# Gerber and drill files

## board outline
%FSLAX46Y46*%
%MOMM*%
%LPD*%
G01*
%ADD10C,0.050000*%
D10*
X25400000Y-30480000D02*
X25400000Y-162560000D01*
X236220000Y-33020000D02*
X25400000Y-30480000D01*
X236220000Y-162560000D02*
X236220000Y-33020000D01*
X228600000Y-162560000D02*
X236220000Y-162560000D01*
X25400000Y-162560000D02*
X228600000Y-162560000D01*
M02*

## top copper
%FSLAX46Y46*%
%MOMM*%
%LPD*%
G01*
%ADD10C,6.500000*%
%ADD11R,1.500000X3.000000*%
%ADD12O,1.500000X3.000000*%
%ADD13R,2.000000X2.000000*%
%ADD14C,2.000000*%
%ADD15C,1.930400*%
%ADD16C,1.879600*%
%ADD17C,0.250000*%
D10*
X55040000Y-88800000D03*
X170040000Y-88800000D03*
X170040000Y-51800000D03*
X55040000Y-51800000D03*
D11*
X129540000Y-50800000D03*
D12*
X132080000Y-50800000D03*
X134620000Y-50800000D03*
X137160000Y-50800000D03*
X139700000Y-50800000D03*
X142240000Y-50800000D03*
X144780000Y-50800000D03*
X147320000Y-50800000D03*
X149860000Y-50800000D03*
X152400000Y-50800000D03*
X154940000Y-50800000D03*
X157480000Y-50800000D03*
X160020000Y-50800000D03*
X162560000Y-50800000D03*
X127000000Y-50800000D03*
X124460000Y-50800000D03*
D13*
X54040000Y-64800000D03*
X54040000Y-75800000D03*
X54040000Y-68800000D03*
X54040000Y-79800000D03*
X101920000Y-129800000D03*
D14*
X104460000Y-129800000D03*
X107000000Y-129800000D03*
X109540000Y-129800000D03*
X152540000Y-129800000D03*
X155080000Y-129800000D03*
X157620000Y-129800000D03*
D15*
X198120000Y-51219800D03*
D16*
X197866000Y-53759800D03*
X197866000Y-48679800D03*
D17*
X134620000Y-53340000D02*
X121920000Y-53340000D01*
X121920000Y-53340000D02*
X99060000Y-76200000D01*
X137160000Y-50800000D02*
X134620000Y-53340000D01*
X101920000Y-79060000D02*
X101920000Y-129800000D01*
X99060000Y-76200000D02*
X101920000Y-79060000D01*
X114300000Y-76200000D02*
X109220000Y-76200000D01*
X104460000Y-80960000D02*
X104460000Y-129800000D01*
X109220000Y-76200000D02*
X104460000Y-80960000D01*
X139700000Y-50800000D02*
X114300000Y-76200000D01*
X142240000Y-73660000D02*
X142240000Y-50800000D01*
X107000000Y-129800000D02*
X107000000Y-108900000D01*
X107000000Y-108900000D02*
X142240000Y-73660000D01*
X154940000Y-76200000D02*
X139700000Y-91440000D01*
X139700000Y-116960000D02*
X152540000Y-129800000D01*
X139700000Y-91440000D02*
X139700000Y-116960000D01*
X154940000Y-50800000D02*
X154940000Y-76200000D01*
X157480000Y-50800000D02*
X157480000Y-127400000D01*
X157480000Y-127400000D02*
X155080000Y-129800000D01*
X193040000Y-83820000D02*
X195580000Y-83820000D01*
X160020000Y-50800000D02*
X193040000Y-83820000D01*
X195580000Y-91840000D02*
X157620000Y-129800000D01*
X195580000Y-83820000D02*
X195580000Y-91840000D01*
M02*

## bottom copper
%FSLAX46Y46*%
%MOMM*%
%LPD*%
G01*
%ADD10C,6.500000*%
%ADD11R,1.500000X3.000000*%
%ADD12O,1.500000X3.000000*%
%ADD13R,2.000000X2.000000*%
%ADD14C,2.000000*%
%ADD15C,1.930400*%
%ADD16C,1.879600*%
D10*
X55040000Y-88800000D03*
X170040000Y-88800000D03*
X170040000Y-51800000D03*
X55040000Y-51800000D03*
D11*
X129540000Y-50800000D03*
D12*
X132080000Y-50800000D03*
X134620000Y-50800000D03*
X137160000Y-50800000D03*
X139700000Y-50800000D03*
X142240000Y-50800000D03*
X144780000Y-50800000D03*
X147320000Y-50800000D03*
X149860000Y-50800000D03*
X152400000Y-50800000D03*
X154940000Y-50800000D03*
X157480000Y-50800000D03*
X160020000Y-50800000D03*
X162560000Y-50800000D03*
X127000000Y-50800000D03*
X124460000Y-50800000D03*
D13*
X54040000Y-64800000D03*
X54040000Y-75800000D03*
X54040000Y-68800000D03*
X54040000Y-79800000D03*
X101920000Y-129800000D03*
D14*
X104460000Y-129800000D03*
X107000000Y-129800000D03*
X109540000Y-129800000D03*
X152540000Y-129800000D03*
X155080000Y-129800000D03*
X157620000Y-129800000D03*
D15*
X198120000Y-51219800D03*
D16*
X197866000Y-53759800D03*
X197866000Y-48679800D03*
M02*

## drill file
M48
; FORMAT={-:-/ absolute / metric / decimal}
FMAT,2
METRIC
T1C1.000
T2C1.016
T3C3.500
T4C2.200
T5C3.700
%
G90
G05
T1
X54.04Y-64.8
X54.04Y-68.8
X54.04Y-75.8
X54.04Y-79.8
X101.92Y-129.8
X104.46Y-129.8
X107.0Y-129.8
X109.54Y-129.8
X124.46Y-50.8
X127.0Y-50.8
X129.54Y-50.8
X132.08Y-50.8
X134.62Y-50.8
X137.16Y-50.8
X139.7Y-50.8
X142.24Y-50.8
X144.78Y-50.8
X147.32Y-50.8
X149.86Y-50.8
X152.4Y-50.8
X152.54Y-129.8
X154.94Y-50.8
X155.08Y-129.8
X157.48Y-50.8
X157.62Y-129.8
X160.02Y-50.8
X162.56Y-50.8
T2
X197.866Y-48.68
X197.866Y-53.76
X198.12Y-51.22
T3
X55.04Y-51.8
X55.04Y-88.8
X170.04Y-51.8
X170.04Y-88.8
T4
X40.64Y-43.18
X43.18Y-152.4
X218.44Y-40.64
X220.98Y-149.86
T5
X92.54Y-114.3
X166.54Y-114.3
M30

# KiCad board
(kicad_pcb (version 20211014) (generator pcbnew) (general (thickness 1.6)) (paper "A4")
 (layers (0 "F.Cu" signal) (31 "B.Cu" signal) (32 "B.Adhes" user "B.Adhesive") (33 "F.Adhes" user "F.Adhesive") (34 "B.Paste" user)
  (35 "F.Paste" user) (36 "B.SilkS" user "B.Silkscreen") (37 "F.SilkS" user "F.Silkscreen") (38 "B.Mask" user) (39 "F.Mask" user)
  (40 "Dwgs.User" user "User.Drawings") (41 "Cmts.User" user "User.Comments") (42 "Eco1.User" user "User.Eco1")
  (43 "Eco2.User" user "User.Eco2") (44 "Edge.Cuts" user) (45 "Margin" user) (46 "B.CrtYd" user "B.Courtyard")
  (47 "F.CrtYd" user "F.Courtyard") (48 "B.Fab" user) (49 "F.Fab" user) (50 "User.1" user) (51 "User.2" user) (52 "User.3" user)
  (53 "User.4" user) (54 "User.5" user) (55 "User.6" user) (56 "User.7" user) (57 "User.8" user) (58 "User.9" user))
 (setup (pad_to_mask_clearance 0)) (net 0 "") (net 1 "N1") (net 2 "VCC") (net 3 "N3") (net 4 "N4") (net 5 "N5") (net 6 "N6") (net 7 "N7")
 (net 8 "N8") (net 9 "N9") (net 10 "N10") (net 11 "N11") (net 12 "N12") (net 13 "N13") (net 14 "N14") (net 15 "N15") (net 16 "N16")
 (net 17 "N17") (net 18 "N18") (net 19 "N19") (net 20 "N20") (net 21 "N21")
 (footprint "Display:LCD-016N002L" (layer "F.Cu") (at 129.54 50.8)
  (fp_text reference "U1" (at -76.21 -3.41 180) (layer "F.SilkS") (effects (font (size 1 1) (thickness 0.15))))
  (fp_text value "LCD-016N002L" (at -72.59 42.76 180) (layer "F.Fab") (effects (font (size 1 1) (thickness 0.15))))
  (pad "" thru_hole circle (at -74.5 38 180) (size 6.5 6.5) (drill 3.5) (layers *.Cu *.Mask))
  (pad "" thru_hole circle (at 40.5 38 180) (size 6.5 6.5) (drill 3.5) (layers *.Cu *.Mask))
  (pad "" thru_hole circle (at 40.5 1 180) (size 6.5 6.5) (drill 3.5) (layers *.Cu *.Mask))
  (pad "" thru_hole circle (at -74.5 1 180) (size 6.5 6.5) (drill 3.5) (layers *.Cu *.Mask))
  (pad "1" thru_hole rect (at 0 0 180) (size 1.5 3) (drill 1) (layers *.Cu *.Mask) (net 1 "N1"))
  (pad "2" thru_hole oval (at 2.54 0 180) (size 1.5 3) (drill 1) (layers *.Cu *.Mask) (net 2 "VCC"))
  (pad "3" thru_hole oval (at 5.08 0 180) (size 1.5 3) (drill 1) (layers *.Cu *.Mask) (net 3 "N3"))
  (pad "4" thru_hole oval (at 7.62 0 180) (size 1.5 3) (drill 1) (layers *.Cu *.Mask) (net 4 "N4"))
  (pad "5" thru_hole oval (at 10.16 0 180) (size 1.5 3) (drill 1) (layers *.Cu *.Mask) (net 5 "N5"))
  (pad "6" thru_hole oval (at 12.7 0 180) (size 1.5 3) (drill 1) (layers *.Cu *.Mask) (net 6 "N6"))
  (pad "7" thru_hole oval (at 15.24 0 180) (size 1.5 3) (drill 1) (layers *.Cu *.Mask) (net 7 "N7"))
  (pad "8" thru_hole oval (at 17.78 0 180) (size 1.5 3) (drill 1) (layers *.Cu *.Mask) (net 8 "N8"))
  (pad "9" thru_hole oval (at 20.32 0 180) (size 1.5 3) (drill 1) (layers *.Cu *.Mask) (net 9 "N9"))
  (pad "10" thru_hole oval (at 22.86 0 180) (size 1.5 3) (drill 1) (layers *.Cu *.Mask) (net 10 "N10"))
  (pad "11" thru_hole oval (at 25.4 0 180) (size 1.5 3) (drill 1) (layers *.Cu *.Mask) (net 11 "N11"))
  (pad "12" thru_hole oval (at 27.94 0 180) (size 1.5 3) (drill 1) (layers *.Cu *.Mask) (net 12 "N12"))
  (pad "13" thru_hole oval (at 30.48 0 180) (size 1.5 3) (drill 1) (layers *.Cu *.Mask) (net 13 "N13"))
  (pad "14" thru_hole oval (at 33.02 0 180) (size 1.5 3) (drill 1) (layers *.Cu *.Mask) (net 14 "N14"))
  (pad "15" thru_hole oval (at -2.54 0 180) (size 1.5 3) (drill 1) (layers *.Cu *.Mask) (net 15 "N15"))
  (pad "16" thru_hole oval (at -5.08 0 180) (size 1.5 3) (drill 1) (layers *.Cu *.Mask) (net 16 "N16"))
  (pad "A1" thru_hole rect (at -75.5 14 180) (size 2 2) (drill 1) (layers *.Cu *.Mask) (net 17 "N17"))
  (pad "A2" thru_hole rect (at -75.5 25 180) (size 2 2) (drill 1) (layers *.Cu *.Mask) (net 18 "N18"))
  (pad "K1" thru_hole rect (at -75.5 18 180) (size 2 2) (drill 1) (layers *.Cu *.Mask) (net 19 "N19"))
  (pad "K2" thru_hole rect (at -75.5 29 180) (size 2 2) (drill 1) (layers *.Cu *.Mask) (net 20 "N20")))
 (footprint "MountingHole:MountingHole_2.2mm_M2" (layer "F.Cu") (at 40.64 43.18)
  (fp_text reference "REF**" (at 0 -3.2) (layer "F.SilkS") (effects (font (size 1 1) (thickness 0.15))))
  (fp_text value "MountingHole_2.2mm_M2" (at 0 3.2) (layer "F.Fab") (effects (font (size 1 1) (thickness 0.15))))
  (pad "" np_thru_hole circle (at 0 0) (size 2.2 2.2) (drill 2.2) (layers *.Cu *.Mask)))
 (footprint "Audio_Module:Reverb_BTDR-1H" (layer "F.Cu") (at 101.92 129.8)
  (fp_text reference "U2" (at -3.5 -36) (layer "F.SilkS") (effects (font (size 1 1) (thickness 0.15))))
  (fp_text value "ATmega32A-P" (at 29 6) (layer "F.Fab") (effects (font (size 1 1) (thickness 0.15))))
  (pad "" np_thru_hole circle (at 64.62 -15.5) (size 3.7 3.7) (drill 3.7) (layers *.Cu *.Mask))
  (pad "" np_thru_hole circle (at -9.38 -15.5) (size 3.7 3.7) (drill 3.7) (layers *.Cu *.Mask))
  (pad "1" thru_hole rect (at 0 0) (size 2 2) (drill 1) (layers *.Cu *.Mask) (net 4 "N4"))
  (pad "2" thru_hole circle (at 2.54 0) (size 2 2) (drill 1) (layers *.Cu *.Mask) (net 5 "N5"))
  (pad "3" thru_hole circle (at 5.08 0) (size 2 2) (drill 1) (layers *.Cu *.Mask) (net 6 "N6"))
  (pad "4" thru_hole circle (at 7.62 0) (size 2 2) (drill 1) (layers *.Cu *.Mask) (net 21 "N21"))
  (pad "5" thru_hole circle (at 50.62 0) (size 2 2) (drill 1) (layers *.Cu *.Mask) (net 11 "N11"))
  (pad "6" thru_hole circle (at 53.16 0) (size 2 2) (drill 1) (layers *.Cu *.Mask) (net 12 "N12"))
  (pad "7" thru_hole circle (at 55.7 0) (size 2 2) (drill 1) (layers *.Cu *.Mask) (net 13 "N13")))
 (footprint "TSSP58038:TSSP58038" (layer "F.Cu") (at 198.12 51.2198)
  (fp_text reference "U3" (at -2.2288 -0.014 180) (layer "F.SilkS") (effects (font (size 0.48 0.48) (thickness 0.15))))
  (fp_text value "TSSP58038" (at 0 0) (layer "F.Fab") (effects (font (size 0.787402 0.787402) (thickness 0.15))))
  (pad "GND" thru_hole circle locked (at 0 0) (size 1.9304 1.9304) (drill 1.016) (layers *.Cu *.Mask))
  (pad "OUT" thru_hole circle locked (at -0.254 2.54) (size 1.8796 1.8796) (drill 1.016) (layers *.Cu *.Mask))
  (pad "VS" thru_hole circle locked (at -0.254 -2.54) (size 1.8796 1.8796) (drill 1.016) (layers *.Cu *.Mask)))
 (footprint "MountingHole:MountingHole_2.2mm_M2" (layer "F.Cu") (at 220.98 149.86)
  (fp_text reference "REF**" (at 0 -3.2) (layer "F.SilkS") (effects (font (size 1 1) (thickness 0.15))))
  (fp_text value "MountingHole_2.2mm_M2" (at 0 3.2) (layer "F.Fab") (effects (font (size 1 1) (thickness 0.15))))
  (pad "" np_thru_hole circle (at 0 0) (size 2.2 2.2) (drill 2.2) (layers *.Cu *.Mask)))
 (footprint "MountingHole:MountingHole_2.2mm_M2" (layer "F.Cu") (at 218.44 40.64)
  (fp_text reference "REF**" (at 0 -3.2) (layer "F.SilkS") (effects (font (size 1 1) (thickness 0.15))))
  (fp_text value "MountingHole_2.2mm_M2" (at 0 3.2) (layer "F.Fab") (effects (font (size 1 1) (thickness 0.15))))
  (pad "" np_thru_hole circle (at 0 0) (size 2.2 2.2) (drill 2.2) (layers *.Cu *.Mask)))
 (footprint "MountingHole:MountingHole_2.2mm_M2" (layer "F.Cu") (at 43.18 152.4)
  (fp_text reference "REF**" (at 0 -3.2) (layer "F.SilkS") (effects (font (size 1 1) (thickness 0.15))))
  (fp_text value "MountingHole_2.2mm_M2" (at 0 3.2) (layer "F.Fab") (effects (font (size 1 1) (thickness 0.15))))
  (pad "" np_thru_hole circle (at 0 0) (size 2.2 2.2) (drill 2.2) (layers *.Cu *.Mask)))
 (gr_line (start 25.4 30.48) (end 25.4 162.56) (layer "Edge.Cuts") (width 0.05))
 (gr_line (start 236.22 33.02) (end 25.4 30.48) (layer "Edge.Cuts") (width 0.05))
 (gr_line (start 236.22 162.56) (end 236.22 33.02) (layer "Edge.Cuts") (width 0.05))
 (gr_line (start 228.6 162.56) (end 236.22 162.56) (layer "Edge.Cuts") (width 0.05))
 (gr_line (start 25.4 162.56) (end 228.6 162.56) (layer "Edge.Cuts") (width 0.05))
 (segment (start 134.62 53.34) (end 121.92 53.34) (width 0.25) (layer "F.Cu") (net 4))
 (segment (start 121.92 53.34) (end 99.06 76.2) (width 0.25) (layer "F.Cu") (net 4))
 (segment (start 137.16 50.8) (end 134.62 53.34) (width 0.25) (layer "F.Cu") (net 4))
 (segment (start 101.92 79.06) (end 101.92 129.8) (width 0.25) (layer "F.Cu") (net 4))
 (segment (start 99.06 76.2) (end 101.92 79.06) (width 0.25) (layer "F.Cu") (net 4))
 (segment (start 114.3 76.2) (end 109.22 76.2) (width 0.25) (layer "F.Cu") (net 5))
 (segment (start 104.46 80.96) (end 104.46 129.8) (width 0.25) (layer "F.Cu") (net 5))
 (segment (start 109.22 76.2) (end 104.46 80.96) (width 0.25) (layer "F.Cu") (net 5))
 (segment (start 139.7 50.8) (end 114.3 76.2) (width 0.25) (layer "F.Cu") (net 5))
 (segment (start 142.24 73.66) (end 142.24 50.8) (width 0.25) (layer "F.Cu") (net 6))
 (segment (start 107 129.8) (end 107 108.9) (width 0.25) (layer "F.Cu") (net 6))
 (segment (start 107 108.9) (end 142.24 73.66) (width 0.25) (layer "F.Cu") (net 6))
 (segment (start 154.94 76.2) (end 139.7 91.44) (width 0.25) (layer "F.Cu") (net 11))
 (segment (start 139.7 116.96) (end 152.54 129.8) (width 0.25) (layer "F.Cu") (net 11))
 (segment (start 139.7 91.44) (end 139.7 116.96) (width 0.25) (layer "F.Cu") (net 11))
 (segment (start 154.94 50.8) (end 154.94 76.2) (width 0.25) (layer "F.Cu") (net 11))
 (segment (start 157.48 50.8) (end 157.48 127.4) (width 0.25) (layer "F.Cu") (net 12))
 (segment (start 157.48 127.4) (end 155.08 129.8) (width 0.25) (layer "F.Cu") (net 12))
 (segment (start 193.04 83.82) (end 195.58 83.82) (width 0.25) (layer "F.Cu") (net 13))
 (segment (start 160.02 50.8) (end 193.04 83.82) (width 0.25) (layer "F.Cu") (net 13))
 (segment (start 195.58 91.84) (end 157.62 129.8) (width 0.25) (layer "F.Cu") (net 13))
 (segment (start 195.58 83.82) (end 195.58 91.84) (width 0.25) (layer "F.Cu") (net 13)))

